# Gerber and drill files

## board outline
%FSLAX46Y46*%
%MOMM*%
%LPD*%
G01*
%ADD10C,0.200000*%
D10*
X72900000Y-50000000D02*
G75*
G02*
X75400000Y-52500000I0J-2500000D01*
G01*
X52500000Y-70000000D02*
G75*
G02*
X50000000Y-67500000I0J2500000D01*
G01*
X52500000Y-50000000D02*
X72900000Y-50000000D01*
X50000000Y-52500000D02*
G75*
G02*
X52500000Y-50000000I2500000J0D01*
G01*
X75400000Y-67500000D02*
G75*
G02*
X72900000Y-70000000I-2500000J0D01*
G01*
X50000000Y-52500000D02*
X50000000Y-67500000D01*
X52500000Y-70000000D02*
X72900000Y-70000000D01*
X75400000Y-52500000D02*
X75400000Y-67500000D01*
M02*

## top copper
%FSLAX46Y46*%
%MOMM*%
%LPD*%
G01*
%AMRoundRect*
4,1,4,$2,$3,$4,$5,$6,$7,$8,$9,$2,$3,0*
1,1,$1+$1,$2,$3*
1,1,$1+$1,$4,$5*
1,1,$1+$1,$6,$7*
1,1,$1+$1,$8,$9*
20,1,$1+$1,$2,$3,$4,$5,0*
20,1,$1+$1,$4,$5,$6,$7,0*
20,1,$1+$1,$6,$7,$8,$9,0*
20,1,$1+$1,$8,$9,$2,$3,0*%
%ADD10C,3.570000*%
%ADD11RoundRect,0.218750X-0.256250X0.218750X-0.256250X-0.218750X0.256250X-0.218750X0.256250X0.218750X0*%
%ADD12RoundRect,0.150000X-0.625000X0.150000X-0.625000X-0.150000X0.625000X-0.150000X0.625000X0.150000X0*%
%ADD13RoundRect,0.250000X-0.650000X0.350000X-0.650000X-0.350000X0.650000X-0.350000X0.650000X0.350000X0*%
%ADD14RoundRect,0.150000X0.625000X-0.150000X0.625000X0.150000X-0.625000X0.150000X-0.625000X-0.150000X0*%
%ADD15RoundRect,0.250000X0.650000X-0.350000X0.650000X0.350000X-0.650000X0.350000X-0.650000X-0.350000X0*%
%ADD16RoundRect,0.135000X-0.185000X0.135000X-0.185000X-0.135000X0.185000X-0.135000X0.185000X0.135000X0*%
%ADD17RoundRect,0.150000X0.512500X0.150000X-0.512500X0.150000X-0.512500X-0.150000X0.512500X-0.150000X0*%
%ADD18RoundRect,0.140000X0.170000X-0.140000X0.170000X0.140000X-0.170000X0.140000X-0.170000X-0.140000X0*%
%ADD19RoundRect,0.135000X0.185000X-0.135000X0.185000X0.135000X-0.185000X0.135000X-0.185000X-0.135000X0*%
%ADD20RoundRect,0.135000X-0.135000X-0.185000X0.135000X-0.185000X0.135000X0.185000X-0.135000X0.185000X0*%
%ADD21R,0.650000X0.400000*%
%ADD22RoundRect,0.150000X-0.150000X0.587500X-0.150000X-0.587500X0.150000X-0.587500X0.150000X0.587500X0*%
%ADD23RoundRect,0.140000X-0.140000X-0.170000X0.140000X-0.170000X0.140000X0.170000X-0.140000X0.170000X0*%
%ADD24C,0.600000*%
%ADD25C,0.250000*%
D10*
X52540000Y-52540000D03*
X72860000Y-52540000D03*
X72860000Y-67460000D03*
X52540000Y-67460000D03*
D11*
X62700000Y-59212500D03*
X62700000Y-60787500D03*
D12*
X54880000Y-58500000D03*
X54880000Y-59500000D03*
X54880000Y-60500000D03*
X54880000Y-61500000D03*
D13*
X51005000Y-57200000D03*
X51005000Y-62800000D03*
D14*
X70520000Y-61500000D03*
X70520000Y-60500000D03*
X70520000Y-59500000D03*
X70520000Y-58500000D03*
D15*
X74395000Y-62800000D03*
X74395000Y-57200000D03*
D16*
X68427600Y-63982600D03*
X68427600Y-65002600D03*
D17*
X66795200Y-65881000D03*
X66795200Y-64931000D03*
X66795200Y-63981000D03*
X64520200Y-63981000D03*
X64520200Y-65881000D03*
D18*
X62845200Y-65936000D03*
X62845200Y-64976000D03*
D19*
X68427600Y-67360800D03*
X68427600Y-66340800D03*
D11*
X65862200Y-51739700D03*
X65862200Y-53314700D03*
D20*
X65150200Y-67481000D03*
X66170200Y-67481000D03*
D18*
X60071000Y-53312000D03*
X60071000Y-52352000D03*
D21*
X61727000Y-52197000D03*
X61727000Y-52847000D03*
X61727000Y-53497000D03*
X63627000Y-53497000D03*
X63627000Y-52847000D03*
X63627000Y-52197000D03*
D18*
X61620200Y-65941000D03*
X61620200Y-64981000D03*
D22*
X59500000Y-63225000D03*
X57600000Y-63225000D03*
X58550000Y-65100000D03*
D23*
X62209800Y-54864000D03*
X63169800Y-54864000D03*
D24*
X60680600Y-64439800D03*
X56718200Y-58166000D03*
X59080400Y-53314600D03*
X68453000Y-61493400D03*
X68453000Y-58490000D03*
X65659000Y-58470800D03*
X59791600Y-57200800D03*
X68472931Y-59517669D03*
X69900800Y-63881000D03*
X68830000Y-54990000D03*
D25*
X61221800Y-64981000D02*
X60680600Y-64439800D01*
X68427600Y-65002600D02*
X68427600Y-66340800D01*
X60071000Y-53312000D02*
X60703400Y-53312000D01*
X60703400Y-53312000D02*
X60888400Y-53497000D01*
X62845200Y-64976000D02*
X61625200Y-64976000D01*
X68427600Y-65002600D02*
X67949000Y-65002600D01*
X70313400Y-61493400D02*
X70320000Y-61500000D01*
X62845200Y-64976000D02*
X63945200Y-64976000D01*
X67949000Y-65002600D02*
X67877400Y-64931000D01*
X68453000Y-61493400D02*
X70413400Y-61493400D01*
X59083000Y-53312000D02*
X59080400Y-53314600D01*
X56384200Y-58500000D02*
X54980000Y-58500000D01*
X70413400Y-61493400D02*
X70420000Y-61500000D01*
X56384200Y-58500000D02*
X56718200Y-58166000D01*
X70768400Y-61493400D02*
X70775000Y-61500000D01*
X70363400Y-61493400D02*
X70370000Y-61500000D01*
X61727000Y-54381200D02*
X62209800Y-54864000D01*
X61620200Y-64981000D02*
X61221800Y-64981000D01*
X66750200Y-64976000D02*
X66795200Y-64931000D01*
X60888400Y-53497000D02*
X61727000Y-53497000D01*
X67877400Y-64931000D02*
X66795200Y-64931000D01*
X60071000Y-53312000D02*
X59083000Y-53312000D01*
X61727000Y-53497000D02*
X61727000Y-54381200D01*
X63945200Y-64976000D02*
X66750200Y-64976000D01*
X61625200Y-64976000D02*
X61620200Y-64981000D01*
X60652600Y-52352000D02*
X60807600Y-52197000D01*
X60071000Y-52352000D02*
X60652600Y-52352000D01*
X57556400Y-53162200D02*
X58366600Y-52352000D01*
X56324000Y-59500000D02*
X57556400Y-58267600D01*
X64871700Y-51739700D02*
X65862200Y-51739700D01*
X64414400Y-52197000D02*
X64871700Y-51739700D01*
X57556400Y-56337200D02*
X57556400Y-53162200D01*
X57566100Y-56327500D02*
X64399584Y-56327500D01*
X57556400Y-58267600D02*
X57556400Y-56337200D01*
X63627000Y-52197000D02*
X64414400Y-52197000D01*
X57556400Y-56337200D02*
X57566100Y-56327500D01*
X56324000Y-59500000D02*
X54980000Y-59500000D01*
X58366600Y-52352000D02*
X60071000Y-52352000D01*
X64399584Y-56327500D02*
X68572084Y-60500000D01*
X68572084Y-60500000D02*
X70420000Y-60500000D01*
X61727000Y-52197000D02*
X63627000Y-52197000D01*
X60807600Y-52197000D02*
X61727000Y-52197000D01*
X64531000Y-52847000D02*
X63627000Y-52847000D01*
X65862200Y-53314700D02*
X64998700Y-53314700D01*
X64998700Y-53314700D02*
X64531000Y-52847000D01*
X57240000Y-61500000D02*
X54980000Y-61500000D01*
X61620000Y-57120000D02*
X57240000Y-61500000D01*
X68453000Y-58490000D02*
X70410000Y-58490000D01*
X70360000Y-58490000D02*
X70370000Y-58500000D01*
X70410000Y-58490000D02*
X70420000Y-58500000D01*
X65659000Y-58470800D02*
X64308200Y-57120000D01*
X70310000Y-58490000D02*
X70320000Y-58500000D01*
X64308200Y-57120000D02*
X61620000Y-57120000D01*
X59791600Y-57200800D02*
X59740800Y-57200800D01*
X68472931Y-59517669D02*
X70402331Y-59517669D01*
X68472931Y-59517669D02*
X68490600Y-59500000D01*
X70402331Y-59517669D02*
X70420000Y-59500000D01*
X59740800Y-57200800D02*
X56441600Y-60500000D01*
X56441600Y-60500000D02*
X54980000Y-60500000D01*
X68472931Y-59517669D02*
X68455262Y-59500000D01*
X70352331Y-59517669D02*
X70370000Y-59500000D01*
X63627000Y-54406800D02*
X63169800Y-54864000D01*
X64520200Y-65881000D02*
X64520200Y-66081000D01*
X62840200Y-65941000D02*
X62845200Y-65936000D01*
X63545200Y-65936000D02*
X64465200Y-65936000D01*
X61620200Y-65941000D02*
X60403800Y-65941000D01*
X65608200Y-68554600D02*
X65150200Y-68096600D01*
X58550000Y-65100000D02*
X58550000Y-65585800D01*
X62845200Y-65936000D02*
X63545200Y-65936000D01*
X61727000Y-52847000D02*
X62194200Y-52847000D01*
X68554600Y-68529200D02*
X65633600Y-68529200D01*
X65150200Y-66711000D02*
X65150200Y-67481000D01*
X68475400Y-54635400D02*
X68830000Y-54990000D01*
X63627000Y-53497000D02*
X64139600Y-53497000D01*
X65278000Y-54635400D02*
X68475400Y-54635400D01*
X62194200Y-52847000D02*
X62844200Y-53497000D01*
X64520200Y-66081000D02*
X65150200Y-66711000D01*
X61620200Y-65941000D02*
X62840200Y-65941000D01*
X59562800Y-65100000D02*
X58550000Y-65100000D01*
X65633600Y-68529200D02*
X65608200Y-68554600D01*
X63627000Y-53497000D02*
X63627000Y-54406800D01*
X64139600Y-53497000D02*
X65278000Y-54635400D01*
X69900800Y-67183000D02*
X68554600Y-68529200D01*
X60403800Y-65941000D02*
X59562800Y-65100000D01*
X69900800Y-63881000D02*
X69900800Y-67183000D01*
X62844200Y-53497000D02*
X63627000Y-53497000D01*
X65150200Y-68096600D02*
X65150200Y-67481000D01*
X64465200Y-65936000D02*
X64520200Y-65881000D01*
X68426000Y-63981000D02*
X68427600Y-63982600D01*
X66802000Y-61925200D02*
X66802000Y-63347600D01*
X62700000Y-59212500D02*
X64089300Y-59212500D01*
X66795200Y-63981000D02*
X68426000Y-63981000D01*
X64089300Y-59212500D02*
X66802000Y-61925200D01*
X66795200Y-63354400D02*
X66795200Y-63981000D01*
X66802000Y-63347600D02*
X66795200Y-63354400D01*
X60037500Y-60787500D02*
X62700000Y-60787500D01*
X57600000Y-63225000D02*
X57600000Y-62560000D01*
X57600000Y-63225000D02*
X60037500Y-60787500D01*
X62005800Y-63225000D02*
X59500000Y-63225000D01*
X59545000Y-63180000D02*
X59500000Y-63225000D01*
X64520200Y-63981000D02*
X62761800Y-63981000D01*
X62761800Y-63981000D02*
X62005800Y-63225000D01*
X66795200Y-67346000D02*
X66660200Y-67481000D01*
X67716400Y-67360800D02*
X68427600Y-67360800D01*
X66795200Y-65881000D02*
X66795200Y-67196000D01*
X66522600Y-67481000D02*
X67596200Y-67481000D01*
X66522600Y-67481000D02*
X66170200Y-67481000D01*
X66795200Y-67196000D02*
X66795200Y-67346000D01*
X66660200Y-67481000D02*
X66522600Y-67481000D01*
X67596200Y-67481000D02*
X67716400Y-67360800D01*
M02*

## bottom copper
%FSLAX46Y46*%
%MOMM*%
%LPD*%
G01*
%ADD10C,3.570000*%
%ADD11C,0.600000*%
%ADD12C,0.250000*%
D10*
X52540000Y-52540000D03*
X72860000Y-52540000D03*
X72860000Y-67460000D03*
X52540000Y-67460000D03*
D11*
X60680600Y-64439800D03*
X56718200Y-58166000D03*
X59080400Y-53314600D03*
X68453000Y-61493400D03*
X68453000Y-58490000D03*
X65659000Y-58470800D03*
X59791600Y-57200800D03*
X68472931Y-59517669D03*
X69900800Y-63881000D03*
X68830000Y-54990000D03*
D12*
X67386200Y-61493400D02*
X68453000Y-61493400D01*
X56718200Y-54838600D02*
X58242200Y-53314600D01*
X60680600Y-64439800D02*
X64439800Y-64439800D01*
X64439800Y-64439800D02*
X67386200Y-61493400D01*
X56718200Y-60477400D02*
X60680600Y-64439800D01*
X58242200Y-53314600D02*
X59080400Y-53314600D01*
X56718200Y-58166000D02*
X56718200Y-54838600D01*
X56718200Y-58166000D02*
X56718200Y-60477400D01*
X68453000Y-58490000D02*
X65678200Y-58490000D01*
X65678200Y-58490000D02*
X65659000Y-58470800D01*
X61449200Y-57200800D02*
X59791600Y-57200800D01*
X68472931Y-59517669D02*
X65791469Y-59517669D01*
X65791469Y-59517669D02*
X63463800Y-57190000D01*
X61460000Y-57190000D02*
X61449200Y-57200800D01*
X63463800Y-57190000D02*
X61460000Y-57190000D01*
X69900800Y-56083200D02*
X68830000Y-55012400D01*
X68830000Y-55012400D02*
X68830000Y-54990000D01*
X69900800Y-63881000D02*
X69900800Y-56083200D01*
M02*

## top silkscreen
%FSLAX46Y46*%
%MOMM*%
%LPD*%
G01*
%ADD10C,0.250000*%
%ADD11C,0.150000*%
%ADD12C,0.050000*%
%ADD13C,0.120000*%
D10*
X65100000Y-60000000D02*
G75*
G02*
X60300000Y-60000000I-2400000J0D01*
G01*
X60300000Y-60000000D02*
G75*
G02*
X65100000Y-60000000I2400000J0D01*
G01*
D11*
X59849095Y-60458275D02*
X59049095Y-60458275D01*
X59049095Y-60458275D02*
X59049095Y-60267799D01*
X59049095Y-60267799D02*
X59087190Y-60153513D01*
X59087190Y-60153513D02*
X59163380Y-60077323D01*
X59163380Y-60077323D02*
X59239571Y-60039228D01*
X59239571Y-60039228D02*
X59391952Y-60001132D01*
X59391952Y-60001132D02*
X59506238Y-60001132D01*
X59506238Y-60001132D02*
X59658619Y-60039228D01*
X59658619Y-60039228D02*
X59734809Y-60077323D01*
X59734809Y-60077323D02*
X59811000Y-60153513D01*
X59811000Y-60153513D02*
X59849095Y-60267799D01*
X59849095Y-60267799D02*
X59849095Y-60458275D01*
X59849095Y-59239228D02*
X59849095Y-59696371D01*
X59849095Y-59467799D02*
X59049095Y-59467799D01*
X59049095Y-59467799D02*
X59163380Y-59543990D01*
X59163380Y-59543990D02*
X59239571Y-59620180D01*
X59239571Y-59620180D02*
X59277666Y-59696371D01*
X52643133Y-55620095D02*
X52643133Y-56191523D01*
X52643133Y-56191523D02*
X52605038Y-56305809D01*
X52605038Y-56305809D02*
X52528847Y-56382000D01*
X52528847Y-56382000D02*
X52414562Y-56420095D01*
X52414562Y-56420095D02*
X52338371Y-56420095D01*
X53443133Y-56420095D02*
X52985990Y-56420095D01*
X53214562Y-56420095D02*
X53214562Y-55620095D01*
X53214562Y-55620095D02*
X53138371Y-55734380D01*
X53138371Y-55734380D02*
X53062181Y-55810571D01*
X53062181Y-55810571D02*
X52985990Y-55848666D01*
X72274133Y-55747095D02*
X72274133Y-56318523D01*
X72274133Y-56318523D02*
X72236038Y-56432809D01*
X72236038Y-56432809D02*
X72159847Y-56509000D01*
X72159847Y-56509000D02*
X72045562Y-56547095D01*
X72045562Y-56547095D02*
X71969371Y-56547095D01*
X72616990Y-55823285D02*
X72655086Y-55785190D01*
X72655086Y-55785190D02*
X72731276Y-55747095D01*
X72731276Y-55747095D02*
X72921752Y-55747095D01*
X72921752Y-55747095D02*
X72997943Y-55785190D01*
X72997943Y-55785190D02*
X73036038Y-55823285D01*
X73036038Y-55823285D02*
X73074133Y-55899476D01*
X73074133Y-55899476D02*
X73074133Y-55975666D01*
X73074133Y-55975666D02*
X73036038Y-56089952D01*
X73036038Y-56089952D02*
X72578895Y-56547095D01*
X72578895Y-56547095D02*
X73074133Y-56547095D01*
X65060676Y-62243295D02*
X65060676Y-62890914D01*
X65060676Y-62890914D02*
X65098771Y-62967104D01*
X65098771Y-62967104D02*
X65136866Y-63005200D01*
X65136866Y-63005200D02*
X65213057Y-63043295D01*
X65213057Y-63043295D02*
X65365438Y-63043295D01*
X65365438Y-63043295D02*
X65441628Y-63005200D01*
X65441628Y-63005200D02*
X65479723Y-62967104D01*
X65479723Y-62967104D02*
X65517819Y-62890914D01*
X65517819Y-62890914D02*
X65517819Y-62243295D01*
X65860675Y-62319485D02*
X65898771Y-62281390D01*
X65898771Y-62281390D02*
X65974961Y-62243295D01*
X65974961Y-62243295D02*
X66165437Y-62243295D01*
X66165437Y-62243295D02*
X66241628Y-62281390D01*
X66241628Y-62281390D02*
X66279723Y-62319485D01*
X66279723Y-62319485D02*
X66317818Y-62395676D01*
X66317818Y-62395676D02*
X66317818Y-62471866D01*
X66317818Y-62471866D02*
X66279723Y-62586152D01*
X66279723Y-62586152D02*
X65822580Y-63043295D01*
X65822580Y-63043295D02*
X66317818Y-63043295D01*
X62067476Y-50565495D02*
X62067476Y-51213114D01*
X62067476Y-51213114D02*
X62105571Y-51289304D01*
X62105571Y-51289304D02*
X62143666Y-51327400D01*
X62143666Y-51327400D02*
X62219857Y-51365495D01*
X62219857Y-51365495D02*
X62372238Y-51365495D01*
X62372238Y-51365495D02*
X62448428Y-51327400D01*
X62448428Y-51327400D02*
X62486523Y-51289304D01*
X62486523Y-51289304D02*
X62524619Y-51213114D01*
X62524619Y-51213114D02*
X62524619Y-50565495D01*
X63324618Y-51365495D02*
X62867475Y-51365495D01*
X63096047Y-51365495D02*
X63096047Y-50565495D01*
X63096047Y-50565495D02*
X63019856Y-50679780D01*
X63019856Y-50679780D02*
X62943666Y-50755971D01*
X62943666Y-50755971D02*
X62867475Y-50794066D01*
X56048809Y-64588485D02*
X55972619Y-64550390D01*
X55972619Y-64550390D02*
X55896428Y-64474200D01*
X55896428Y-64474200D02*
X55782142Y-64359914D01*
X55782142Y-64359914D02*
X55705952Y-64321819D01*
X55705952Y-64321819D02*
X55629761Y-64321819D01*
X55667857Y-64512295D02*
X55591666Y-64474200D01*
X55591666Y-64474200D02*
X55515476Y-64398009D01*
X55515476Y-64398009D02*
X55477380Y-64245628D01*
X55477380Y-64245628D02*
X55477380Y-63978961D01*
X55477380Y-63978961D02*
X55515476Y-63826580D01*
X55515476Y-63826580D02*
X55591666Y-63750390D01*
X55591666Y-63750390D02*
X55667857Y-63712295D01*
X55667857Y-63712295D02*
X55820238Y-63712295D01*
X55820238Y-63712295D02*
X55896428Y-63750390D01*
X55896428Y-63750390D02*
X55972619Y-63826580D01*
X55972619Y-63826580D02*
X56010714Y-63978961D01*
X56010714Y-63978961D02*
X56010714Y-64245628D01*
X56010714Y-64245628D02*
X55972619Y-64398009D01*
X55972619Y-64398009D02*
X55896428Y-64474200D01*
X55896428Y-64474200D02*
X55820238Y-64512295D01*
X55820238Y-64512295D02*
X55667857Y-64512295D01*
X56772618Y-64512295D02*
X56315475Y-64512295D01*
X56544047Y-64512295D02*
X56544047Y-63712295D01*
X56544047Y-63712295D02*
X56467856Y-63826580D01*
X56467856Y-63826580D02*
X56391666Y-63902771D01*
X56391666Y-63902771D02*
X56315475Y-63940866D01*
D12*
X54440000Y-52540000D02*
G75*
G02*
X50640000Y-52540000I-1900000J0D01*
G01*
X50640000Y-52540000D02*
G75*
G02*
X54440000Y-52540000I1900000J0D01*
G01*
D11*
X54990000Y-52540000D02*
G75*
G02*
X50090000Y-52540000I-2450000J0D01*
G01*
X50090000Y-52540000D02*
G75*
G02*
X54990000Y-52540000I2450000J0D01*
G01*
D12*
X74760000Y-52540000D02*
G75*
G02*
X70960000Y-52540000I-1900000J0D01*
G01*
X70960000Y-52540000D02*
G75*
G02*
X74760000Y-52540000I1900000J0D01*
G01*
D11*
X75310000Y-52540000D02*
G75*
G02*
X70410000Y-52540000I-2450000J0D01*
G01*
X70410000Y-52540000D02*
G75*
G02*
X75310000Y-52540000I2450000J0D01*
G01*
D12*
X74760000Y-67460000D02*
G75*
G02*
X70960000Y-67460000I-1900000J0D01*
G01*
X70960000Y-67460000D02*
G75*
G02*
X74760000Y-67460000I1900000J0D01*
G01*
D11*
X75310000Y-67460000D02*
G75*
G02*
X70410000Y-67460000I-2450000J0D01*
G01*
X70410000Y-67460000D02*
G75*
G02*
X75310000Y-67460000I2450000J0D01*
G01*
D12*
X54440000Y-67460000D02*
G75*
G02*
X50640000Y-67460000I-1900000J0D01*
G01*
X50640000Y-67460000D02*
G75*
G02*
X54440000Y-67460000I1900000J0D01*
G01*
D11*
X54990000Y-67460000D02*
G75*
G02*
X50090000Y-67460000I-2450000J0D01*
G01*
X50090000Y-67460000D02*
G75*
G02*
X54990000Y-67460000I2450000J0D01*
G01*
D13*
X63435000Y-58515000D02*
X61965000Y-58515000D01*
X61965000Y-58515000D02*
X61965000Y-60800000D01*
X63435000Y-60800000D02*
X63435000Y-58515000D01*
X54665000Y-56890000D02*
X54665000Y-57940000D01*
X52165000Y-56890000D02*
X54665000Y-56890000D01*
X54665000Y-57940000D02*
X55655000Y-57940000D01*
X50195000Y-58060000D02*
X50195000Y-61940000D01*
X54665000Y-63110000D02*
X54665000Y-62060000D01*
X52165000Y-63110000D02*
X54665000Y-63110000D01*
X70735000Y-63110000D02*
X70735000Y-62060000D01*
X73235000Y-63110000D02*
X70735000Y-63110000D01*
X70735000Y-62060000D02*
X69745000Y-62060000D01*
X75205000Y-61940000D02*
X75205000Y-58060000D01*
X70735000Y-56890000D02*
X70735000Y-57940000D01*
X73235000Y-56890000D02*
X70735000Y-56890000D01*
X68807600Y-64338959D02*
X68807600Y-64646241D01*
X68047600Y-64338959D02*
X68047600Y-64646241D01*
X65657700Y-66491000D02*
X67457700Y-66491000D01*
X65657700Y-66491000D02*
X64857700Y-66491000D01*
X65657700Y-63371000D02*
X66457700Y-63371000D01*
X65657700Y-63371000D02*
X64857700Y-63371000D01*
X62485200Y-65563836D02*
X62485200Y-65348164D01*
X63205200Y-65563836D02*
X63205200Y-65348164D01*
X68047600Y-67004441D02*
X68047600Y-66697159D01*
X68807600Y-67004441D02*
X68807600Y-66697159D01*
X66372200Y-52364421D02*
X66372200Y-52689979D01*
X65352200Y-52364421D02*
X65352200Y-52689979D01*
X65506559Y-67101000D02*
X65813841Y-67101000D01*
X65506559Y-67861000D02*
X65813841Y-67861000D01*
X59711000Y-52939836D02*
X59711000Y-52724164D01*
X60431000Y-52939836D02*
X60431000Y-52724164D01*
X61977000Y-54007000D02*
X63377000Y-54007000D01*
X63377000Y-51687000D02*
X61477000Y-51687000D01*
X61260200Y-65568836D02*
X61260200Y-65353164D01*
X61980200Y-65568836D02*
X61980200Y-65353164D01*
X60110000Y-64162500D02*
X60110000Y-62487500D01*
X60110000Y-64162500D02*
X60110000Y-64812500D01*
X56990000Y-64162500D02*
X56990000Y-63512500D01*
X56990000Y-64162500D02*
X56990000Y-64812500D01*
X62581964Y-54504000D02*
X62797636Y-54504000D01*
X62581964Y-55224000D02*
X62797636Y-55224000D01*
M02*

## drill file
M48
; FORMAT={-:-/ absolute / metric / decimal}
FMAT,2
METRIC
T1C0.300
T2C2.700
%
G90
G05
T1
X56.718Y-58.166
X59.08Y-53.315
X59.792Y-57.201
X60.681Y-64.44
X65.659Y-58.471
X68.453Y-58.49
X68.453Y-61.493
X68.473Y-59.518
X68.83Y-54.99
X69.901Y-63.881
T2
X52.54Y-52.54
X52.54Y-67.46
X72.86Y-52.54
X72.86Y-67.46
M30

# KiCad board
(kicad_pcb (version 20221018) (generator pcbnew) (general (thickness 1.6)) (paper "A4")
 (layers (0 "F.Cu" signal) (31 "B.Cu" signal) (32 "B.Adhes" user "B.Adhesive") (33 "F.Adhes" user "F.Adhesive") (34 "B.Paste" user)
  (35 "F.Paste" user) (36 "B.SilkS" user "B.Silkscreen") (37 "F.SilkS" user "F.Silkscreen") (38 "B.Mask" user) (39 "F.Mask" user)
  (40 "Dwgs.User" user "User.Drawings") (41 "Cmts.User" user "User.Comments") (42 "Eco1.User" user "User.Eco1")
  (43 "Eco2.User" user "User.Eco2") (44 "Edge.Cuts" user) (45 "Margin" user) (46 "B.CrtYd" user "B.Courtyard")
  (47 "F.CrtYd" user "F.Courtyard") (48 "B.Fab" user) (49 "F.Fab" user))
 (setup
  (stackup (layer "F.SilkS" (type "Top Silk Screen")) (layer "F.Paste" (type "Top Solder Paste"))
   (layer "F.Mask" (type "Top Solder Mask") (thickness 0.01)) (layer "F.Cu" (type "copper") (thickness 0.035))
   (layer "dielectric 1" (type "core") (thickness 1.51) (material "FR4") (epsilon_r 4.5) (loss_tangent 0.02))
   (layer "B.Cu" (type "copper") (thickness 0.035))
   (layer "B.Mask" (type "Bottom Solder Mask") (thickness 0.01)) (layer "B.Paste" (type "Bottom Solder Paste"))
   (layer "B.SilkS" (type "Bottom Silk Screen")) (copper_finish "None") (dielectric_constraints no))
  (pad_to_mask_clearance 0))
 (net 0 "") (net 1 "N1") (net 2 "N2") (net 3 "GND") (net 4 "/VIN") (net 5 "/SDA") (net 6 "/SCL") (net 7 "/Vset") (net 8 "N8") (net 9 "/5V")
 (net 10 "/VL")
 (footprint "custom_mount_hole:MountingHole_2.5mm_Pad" (layer "F.Cu") (at 52.54 52.54)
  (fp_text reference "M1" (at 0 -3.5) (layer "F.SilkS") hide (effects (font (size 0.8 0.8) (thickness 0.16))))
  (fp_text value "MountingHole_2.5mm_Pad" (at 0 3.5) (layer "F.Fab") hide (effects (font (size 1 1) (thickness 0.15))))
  (fp_circle (center 0 0) (end 1.9 0) (stroke (width 0.05) (type solid)) (fill none) (layer "F.SilkS"))
  (fp_circle (center 0 0) (end 2.45 0) (stroke (width 0.15) (type solid)) (fill none) (layer "F.SilkS"))
  (pad "~" thru_hole circle (at 0 0) (size 3.57 3.57) (drill 2.7) (layers "*.Cu" "*.Mask")))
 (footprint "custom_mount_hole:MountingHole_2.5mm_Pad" (layer "F.Cu") (at 72.86 52.54)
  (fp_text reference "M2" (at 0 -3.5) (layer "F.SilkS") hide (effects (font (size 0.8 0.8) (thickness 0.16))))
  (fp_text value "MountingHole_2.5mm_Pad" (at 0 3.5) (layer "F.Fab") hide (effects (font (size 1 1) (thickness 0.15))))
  (fp_circle (center 0 0) (end 1.9 0) (stroke (width 0.05) (type solid)) (fill none) (layer "F.SilkS"))
  (fp_circle (center 0 0) (end 2.45 0) (stroke (width 0.15) (type solid)) (fill none) (layer "F.SilkS"))
  (pad "~" thru_hole circle (at 0 0) (size 3.57 3.57) (drill 2.7) (layers "*.Cu" "*.Mask")))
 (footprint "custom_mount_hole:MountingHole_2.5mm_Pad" (layer "F.Cu") (at 72.86 67.46)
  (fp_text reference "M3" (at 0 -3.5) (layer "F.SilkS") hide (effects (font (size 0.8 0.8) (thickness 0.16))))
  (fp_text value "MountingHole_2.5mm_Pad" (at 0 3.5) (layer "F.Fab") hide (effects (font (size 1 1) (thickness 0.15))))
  (fp_circle (center 0 0) (end 1.9 0) (stroke (width 0.05) (type solid)) (fill none) (layer "F.SilkS"))
  (fp_circle (center 0 0) (end 2.45 0) (stroke (width 0.15) (type solid)) (fill none) (layer "F.SilkS"))
  (pad "~" thru_hole circle (at 0 0) (size 3.57 3.57) (drill 2.7) (layers "*.Cu" "*.Mask")))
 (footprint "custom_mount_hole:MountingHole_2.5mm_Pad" (layer "F.Cu") (at 52.54 67.46)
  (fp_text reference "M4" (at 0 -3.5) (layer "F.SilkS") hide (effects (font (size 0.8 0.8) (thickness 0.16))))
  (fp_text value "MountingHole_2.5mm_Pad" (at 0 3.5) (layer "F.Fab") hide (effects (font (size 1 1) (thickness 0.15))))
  (fp_circle (center 0 0) (end 1.9 0) (stroke (width 0.05) (type solid)) (fill none) (layer "F.SilkS"))
  (fp_circle (center 0 0) (end 2.45 0) (stroke (width 0.15) (type solid)) (fill none) (layer "F.SilkS"))
  (pad "~" thru_hole circle (at 0 0) (size 3.57 3.57) (drill 2.7) (layers "*.Cu" "*.Mask")))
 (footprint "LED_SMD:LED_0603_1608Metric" (layer "F.Cu") (at 62.7 60 -90)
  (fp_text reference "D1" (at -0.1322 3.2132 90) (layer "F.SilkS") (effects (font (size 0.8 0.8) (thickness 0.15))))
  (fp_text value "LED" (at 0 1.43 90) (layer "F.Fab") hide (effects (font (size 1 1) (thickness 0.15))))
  (fp_line (start -1.485 -0.735) (end -1.485 0.735) (stroke (width 0.12) (type solid)) (layer "F.SilkS"))
  (fp_line (start -1.485 0.735) (end 0.8 0.735) (stroke (width 0.12) (type solid)) (layer "F.SilkS"))
  (fp_line (start 0.8 -0.735) (end -1.485 -0.735) (stroke (width 0.12) (type solid)) (layer "F.SilkS"))
  (pad "1" smd roundrect (at -0.7875 0 270) (size 0.875 0.95) (layers "F.Cu" "F.Paste" "F.Mask") (roundrect_rratio 0.25) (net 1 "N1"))
  (pad "2" smd roundrect (at 0.7875 0 270) (size 0.875 0.95) (layers "F.Cu" "F.Paste" "F.Mask") (roundrect_rratio 0.25) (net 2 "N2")))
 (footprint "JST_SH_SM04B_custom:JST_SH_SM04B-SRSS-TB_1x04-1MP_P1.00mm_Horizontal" (layer "F.Cu") (at 52.88 60 -90)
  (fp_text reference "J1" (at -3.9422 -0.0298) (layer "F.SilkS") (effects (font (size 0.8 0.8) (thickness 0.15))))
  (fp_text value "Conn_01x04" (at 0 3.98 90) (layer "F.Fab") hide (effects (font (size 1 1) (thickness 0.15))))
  (fp_line (start -3.11 -1.785) (end -2.06 -1.785) (stroke (width 0.12) (type solid)) (layer "F.SilkS"))
  (fp_line (start -3.11 0.715) (end -3.11 -1.785) (stroke (width 0.12) (type solid)) (layer "F.SilkS"))
  (fp_line (start -2.06 -1.785) (end -2.06 -2.775) (stroke (width 0.12) (type solid)) (layer "F.SilkS"))
  (fp_line (start -1.94 2.685) (end 1.94 2.685) (stroke (width 0.12) (type solid)) (layer "F.SilkS"))
  (fp_line (start 3.11 -1.785) (end 2.06 -1.785) (stroke (width 0.12) (type solid)) (layer "F.SilkS"))
  (fp_line (start 3.11 0.715) (end 3.11 -1.785) (stroke (width 0.12) (type solid)) (layer "F.SilkS"))
  (pad "1" smd roundrect (at -1.5 -2 270) (size 0.6 1.55) (layers "F.Cu" "F.Paste" "F.Mask") (roundrect_rratio 0.25) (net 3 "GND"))
  (pad "2" smd roundrect (at -0.5 -2 270) (size 0.6 1.55) (layers "F.Cu" "F.Paste" "F.Mask") (roundrect_rratio 0.25) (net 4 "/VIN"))
  (pad "3" smd roundrect (at 0.5 -2 270) (size 0.6 1.55) (layers "F.Cu" "F.Paste" "F.Mask") (roundrect_rratio 0.25) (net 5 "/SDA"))
  (pad "4" smd roundrect (at 1.5 -2 270) (size 0.6 1.55) (layers "F.Cu" "F.Paste" "F.Mask") (roundrect_rratio 0.25) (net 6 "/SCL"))
  (pad "MP" smd roundrect (at -2.8 1.875 270) (size 1.2 1.8) (layers "F.Cu" "F.Paste" "F.Mask") (roundrect_rratio 0.2083333333))
  (pad "MP" smd roundrect (at 2.8 1.875 270) (size 1.2 1.8) (layers "F.Cu" "F.Paste" "F.Mask") (roundrect_rratio 0.2083333333)))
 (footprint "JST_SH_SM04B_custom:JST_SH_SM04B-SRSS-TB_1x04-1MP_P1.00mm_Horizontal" (layer "F.Cu") (at 72.52 60 90)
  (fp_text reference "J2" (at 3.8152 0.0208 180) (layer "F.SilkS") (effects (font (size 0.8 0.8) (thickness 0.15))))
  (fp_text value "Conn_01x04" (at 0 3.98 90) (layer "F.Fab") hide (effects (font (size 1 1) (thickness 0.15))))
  (fp_line (start -3.11 -1.785) (end -2.06 -1.785) (stroke (width 0.12) (type solid)) (layer "F.SilkS"))
  (fp_line (start -3.11 0.715) (end -3.11 -1.785) (stroke (width 0.12) (type solid)) (layer "F.SilkS"))
  (fp_line (start -2.06 -1.785) (end -2.06 -2.775) (stroke (width 0.12) (type solid)) (layer "F.SilkS"))
  (fp_line (start -1.94 2.685) (end 1.94 2.685) (stroke (width 0.12) (type solid)) (layer "F.SilkS"))
  (fp_line (start 3.11 -1.785) (end 2.06 -1.785) (stroke (width 0.12) (type solid)) (layer "F.SilkS"))
  (fp_line (start 3.11 0.715) (end 3.11 -1.785) (stroke (width 0.12) (type solid)) (layer "F.SilkS"))
  (pad "1" smd roundrect (at -1.5 -2 90) (size 0.6 1.55) (layers "F.Cu" "F.Paste" "F.Mask") (roundrect_rratio 0.25) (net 3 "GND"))
  (pad "2" smd roundrect (at -0.5 -2 90) (size 0.6 1.55) (layers "F.Cu" "F.Paste" "F.Mask") (roundrect_rratio 0.25) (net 4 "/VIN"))
  (pad "3" smd roundrect (at 0.5 -2 90) (size 0.6 1.55) (layers "F.Cu" "F.Paste" "F.Mask") (roundrect_rratio 0.25) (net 5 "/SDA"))
  (pad "4" smd roundrect (at 1.5 -2 90) (size 0.6 1.55) (layers "F.Cu" "F.Paste" "F.Mask") (roundrect_rratio 0.25) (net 6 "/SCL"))
  (pad "MP" smd roundrect (at -2.8 1.875 90) (size 1.2 1.8) (layers "F.Cu" "F.Paste" "F.Mask") (roundrect_rratio 0.2083333333))
  (pad "MP" smd roundrect (at 2.8 1.875 90) (size 1.2 1.8) (layers "F.Cu" "F.Paste" "F.Mask") (roundrect_rratio 0.2083333333)))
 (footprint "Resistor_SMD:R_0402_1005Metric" (layer "F.Cu") (at 68.4276 64.4926 -90)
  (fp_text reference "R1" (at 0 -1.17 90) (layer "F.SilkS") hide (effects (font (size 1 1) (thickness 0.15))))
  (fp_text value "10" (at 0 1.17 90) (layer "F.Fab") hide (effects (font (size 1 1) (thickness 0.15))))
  (fp_line (start -0.153641 -0.38) (end 0.153641 -0.38) (stroke (width 0.12) (type solid)) (layer "F.SilkS"))
  (fp_line (start -0.153641 0.38) (end 0.153641 0.38) (stroke (width 0.12) (type solid)) (layer "F.SilkS"))
  (pad "1" smd roundrect (at -0.51 0 270) (size 0.54 0.64) (layers "F.Cu" "F.Paste" "F.Mask") (roundrect_rratio 0.25) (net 1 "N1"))
  (pad "2" smd roundrect (at 0.51 0 270) (size 0.54 0.64) (layers "F.Cu" "F.Paste" "F.Mask") (roundrect_rratio 0.25) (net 3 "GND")))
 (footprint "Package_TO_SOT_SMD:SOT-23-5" (layer "F.Cu") (at 65.6577 64.931 180)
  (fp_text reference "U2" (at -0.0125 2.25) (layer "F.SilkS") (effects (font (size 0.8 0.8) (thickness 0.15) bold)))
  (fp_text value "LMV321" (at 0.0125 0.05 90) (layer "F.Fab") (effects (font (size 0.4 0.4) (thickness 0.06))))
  (fp_line (start 0 -1.56) (end -1.8 -1.56) (stroke (width 0.12) (type solid)) (layer "F.SilkS"))
  (fp_line (start 0 -1.56) (end 0.8 -1.56) (stroke (width 0.12) (type solid)) (layer "F.SilkS"))
  (fp_line (start 0 1.56) (end -0.8 1.56) (stroke (width 0.12) (type solid)) (layer "F.SilkS"))
  (fp_line (start 0 1.56) (end 0.8 1.56) (stroke (width 0.12) (type solid)) (layer "F.SilkS"))
  (pad "1" smd roundrect (at -1.1375 -0.95 180) (size 1.325 0.6) (layers "F.Cu" "F.Paste" "F.Mask") (roundrect_rratio 0.25) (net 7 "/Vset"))
  (pad "2" smd roundrect (at -1.1375 0 180) (size 1.325 0.6) (layers "F.Cu" "F.Paste" "F.Mask") (roundrect_rratio 0.25) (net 3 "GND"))
  (pad "3" smd roundrect (at -1.1375 0.95 180) (size 1.325 0.6) (layers "F.Cu" "F.Paste" "F.Mask") (roundrect_rratio 0.25) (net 1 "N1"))
  (pad "4" smd roundrect (at 1.1375 0.95 180) (size 1.325 0.6) (layers "F.Cu" "F.Paste" "F.Mask") (roundrect_rratio 0.25) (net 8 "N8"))
  (pad "5" smd roundrect (at 1.1375 -0.95 180) (size 1.325 0.6) (layers "F.Cu" "F.Paste" "F.Mask") (roundrect_rratio 0.25) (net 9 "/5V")))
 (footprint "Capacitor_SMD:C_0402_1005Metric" (layer "F.Cu") (at 62.8452 65.456 90)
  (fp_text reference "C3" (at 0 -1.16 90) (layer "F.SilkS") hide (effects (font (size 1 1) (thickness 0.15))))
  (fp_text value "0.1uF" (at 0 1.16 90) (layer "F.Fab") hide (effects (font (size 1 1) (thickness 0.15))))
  (fp_line (start -0.107836 -0.36) (end 0.107836 -0.36) (stroke (width 0.12) (type solid)) (layer "F.SilkS"))
  (fp_line (start -0.107836 0.36) (end 0.107836 0.36) (stroke (width 0.12) (type solid)) (layer "F.SilkS"))
  (pad "1" smd roundrect (at -0.48 0 90) (size 0.56 0.62) (layers "F.Cu" "F.Paste" "F.Mask") (roundrect_rratio 0.25) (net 9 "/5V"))
  (pad "2" smd roundrect (at 0.48 0 90) (size 0.56 0.62) (layers "F.Cu" "F.Paste" "F.Mask") (roundrect_rratio 0.25) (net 3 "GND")))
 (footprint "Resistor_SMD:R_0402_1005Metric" (layer "F.Cu") (at 68.4276 66.8508 90)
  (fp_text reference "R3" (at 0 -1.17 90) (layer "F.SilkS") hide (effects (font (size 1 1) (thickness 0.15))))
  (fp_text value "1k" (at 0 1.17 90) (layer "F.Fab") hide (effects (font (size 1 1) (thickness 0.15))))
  (fp_line (start -0.153641 -0.38) (end 0.153641 -0.38) (stroke (width 0.12) (type solid)) (layer "F.SilkS"))
  (fp_line (start -0.153641 0.38) (end 0.153641 0.38) (stroke (width 0.12) (type solid)) (layer "F.SilkS"))
  (pad "1" smd roundrect (at -0.51 0 90) (size 0.54 0.64) (layers "F.Cu" "F.Paste" "F.Mask") (roundrect_rratio 0.25) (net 7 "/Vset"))
  (pad "2" smd roundrect (at 0.51 0 90) (size 0.54 0.64) (layers "F.Cu" "F.Paste" "F.Mask") (roundrect_rratio 0.25) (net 3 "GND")))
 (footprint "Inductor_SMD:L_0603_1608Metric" (layer "F.Cu") (at 65.8622 52.5272 -90)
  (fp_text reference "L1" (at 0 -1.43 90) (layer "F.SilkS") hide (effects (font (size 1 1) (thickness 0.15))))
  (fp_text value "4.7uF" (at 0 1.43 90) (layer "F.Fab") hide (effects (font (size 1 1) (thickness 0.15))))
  (fp_line (start -0.162779 -0.51) (end 0.162779 -0.51) (stroke (width 0.12) (type solid)) (layer "F.SilkS"))
  (fp_line (start -0.162779 0.51) (end 0.162779 0.51) (stroke (width 0.12) (type solid)) (layer "F.SilkS"))
  (pad "1" smd roundrect (at -0.7875 0 270) (size 0.875 0.95) (layers "F.Cu" "F.Paste" "F.Mask") (roundrect_rratio 0.25) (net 4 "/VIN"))
  (pad "2" smd roundrect (at 0.7875 0 270) (size 0.875 0.95) (layers "F.Cu" "F.Paste" "F.Mask") (roundrect_rratio 0.25) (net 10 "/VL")))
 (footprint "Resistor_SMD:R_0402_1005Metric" (layer "F.Cu") (at 65.6602 67.481)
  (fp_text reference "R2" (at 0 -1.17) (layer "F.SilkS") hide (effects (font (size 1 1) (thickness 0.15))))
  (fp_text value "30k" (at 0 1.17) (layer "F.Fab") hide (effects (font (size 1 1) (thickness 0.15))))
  (fp_line (start -0.153641 -0.38) (end 0.153641 -0.38) (stroke (width 0.12) (type solid)) (layer "F.SilkS"))
  (fp_line (start -0.153641 0.38) (end 0.153641 0.38) (stroke (width 0.12) (type solid)) (layer "F.SilkS"))
  (pad "1" smd roundrect (at -0.51 0) (size 0.54 0.64) (layers "F.Cu" "F.Paste" "F.Mask") (roundrect_rratio 0.25) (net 9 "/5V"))
  (pad "2" smd roundrect (at 0.51 0) (size 0.54 0.64) (layers "F.Cu" "F.Paste" "F.Mask") (roundrect_rratio 0.25) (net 7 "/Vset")))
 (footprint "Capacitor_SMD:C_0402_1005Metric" (layer "F.Cu") (at 60.071 52.832 90)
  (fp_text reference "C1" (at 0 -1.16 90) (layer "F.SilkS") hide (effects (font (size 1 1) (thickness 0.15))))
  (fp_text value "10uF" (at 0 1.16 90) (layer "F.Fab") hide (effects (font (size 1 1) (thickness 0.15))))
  (fp_line (start -0.107836 -0.36) (end 0.107836 -0.36) (stroke (width 0.12) (type solid)) (layer "F.SilkS"))
  (fp_line (start -0.107836 0.36) (end 0.107836 0.36) (stroke (width 0.12) (type solid)) (layer "F.SilkS"))
  (pad "1" smd roundrect (at -0.48 0 90) (size 0.56 0.62) (layers "F.Cu" "F.Paste" "F.Mask") (roundrect_rratio 0.25) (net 3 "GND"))
  (pad "2" smd roundrect (at 0.48 0 90) (size 0.56 0.62) (layers "F.Cu" "F.Paste" "F.Mask") (roundrect_rratio 0.25) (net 4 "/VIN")))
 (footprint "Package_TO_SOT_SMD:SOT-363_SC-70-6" (layer "F.Cu") (at 62.677 52.847)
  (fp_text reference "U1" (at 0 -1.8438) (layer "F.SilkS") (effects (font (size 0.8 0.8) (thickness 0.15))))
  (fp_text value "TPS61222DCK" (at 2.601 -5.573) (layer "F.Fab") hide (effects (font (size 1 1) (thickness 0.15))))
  (fp_line (start -0.7 1.16) (end 0.7 1.16) (stroke (width 0.12) (type solid)) (layer "F.SilkS"))
  (fp_line (start 0.7 -1.16) (end -1.2 -1.16) (stroke (width 0.12) (type solid)) (layer "F.SilkS"))
  (pad "1" smd rect (at -0.95 -0.65) (size 0.65 0.4) (layers "F.Cu" "F.Paste" "F.Mask") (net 4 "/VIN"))
  (pad "2" smd rect (at -0.95 0) (size 0.65 0.4) (layers "F.Cu" "F.Paste" "F.Mask") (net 9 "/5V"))
  (pad "3" smd rect (at -0.95 0.65) (size 0.65 0.4) (layers "F.Cu" "F.Paste" "F.Mask") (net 3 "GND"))
  (pad "4" smd rect (at 0.95 0.65) (size 0.65 0.4) (layers "F.Cu" "F.Paste" "F.Mask") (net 9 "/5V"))
  (pad "5" smd rect (at 0.95 0) (size 0.65 0.4) (layers "F.Cu" "F.Paste" "F.Mask") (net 10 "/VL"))
  (pad "6" smd rect (at 0.95 -0.65) (size 0.65 0.4) (layers "F.Cu" "F.Paste" "F.Mask") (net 4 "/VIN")))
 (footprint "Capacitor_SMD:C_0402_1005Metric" (layer "F.Cu") (at 61.6202 65.461 90)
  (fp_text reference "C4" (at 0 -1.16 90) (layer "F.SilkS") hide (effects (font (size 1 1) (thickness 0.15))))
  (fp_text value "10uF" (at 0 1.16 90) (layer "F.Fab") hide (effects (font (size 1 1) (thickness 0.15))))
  (fp_line (start -0.107836 -0.36) (end 0.107836 -0.36) (stroke (width 0.12) (type solid)) (layer "F.SilkS"))
  (fp_line (start -0.107836 0.36) (end 0.107836 0.36) (stroke (width 0.12) (type solid)) (layer "F.SilkS"))
  (pad "1" smd roundrect (at -0.48 0 90) (size 0.56 0.62) (layers "F.Cu" "F.Paste" "F.Mask") (roundrect_rratio 0.25) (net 9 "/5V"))
  (pad "2" smd roundrect (at 0.48 0 90) (size 0.56 0.62) (layers "F.Cu" "F.Paste" "F.Mask") (roundrect_rratio 0.25) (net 3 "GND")))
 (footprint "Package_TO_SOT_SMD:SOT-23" (layer "F.Cu") (at 58.55 64.1625 -90)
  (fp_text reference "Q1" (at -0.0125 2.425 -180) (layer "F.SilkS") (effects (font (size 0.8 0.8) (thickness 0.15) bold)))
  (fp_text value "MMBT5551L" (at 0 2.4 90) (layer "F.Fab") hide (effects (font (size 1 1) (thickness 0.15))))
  (fp_line (start 0 -1.56) (end -1.675 -1.56) (stroke (width 0.12) (type solid)) (layer "F.SilkS"))
  (fp_line (start 0 -1.56) (end 0.65 -1.56) (stroke (width 0.12) (type solid)) (layer "F.SilkS"))
  (fp_line (start 0 1.56) (end -0.65 1.56) (stroke (width 0.12) (type solid)) (layer "F.SilkS"))
  (fp_line (start 0 1.56) (end 0.65 1.56) (stroke (width 0.12) (type solid)) (layer "F.SilkS"))
  (pad "1" smd roundrect (at -0.9375 -0.95 270) (size 1.475 0.6) (layers "F.Cu" "F.Paste" "F.Mask") (roundrect_rratio 0.25) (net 8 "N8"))
  (pad "2" smd roundrect (at -0.9375 0.95 270) (size 1.475 0.6) (layers "F.Cu" "F.Paste" "F.Mask") (roundrect_rratio 0.25) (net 2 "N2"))
  (pad "3" smd roundrect (at 0.9375 0 270) (size 1.475 0.6) (layers "F.Cu" "F.Paste" "F.Mask") (roundrect_rratio 0.25) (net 9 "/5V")))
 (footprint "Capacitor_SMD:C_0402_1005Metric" (layer "F.Cu") (at 62.6898 54.864)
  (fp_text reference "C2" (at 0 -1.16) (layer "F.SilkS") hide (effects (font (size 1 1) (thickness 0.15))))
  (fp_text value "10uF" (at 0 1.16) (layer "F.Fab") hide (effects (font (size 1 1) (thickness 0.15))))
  (fp_line (start -0.107836 -0.36) (end 0.107836 -0.36) (stroke (width 0.12) (type solid)) (layer "F.SilkS"))
  (fp_line (start -0.107836 0.36) (end 0.107836 0.36) (stroke (width 0.12) (type solid)) (layer "F.SilkS"))
  (pad "1" smd roundrect (at -0.48 0) (size 0.56 0.62) (layers "F.Cu" "F.Paste" "F.Mask") (roundrect_rratio 0.25) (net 3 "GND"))
  (pad "2" smd roundrect (at 0.48 0) (size 0.56 0.62) (layers "F.Cu" "F.Paste" "F.Mask") (roundrect_rratio 0.25) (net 9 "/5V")))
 (gr_circle (center 62.7 60) (end 65.1 60) (stroke (width 0.25) (type solid)) (fill none) (layer "F.SilkS"))
 (gr_arc (start 72.9 50) (mid 74.667767 50.732233) (end 75.4 52.5) (stroke (width 0.2) (type solid)) (layer "Edge.Cuts"))
 (gr_arc (start 52.5 70) (mid 50.732233 69.267767) (end 50 67.5) (stroke (width 0.2) (type solid)) (layer "Edge.Cuts"))
 (gr_line (start 52.5 50) (end 72.9 50) (stroke (width 0.2) (type solid)) (layer "Edge.Cuts"))
 (gr_arc (start 50 52.5) (mid 50.732233 50.732233) (end 52.5 50) (stroke (width 0.2) (type solid)) (layer "Edge.Cuts"))
 (gr_arc (start 75.4 67.5) (mid 74.667767 69.267767) (end 72.9 70) (stroke (width 0.2) (type solid)) (layer "Edge.Cuts"))
 (gr_line (start 50 52.5) (end 50 67.5) (stroke (width 0.2) (type solid)) (layer "Edge.Cuts"))
 (gr_line (start 52.5 70) (end 72.9 70) (stroke (width 0.2) (type solid)) (layer "Edge.Cuts"))
 (gr_line (start 75.4 52.5) (end 75.4 67.5) (stroke (width 0.2) (type solid)) (layer "Edge.Cuts"))
 (segment (start 61.2218 64.981) (end 60.6806 64.4398) (width 0.25) (layer "F.Cu") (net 3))
 (segment (start 68.4276 65.0026) (end 68.4276 66.3408) (width 0.25) (layer "F.Cu") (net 3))
 (segment (start 60.071 53.312) (end 60.7034 53.312) (width 0.25) (layer "F.Cu") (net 3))
 (segment (start 60.7034 53.312) (end 60.8884 53.497) (width 0.25) (layer "F.Cu") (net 3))
 (segment (start 62.8452 64.976) (end 61.6252 64.976) (width 0.25) (layer "F.Cu") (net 3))
 (segment (start 68.4276 65.0026) (end 67.949 65.0026) (width 0.25) (layer "F.Cu") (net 3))
 (segment (start 70.3134 61.4934) (end 70.32 61.5) (width 0.25) (layer "F.Cu") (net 3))
 (segment (start 62.8452 64.976) (end 63.9452 64.976) (width 0.25) (layer "F.Cu") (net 3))
 (segment (start 67.949 65.0026) (end 67.8774 64.931) (width 0.25) (layer "F.Cu") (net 3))
 (segment (start 68.453 61.4934) (end 70.4134 61.4934) (width 0.25) (layer "F.Cu") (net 3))
 (segment (start 59.083 53.312) (end 59.0804 53.3146) (width 0.25) (layer "F.Cu") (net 3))
 (segment (start 56.3842 58.5) (end 54.98 58.5) (width 0.25) (layer "F.Cu") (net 3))
 (segment (start 70.4134 61.4934) (end 70.42 61.5) (width 0.25) (layer "F.Cu") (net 3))
 (segment (start 56.3842 58.5) (end 56.7182 58.166) (width 0.25) (layer "F.Cu") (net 3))
 (segment (start 70.7684 61.4934) (end 70.775 61.5) (width 0.25) (layer "F.Cu") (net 3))
 (segment (start 70.3634 61.4934) (end 70.37 61.5) (width 0.25) (layer "F.Cu") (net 3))
 (segment (start 61.727 54.3812) (end 62.2098 54.864) (width 0.25) (layer "F.Cu") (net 3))
 (segment (start 61.6202 64.981) (end 61.2218 64.981) (width 0.25) (layer "F.Cu") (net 3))
 (segment (start 66.7502 64.976) (end 66.7952 64.931) (width 0.25) (layer "F.Cu") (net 3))
 (segment (start 60.8884 53.497) (end 61.727 53.497) (width 0.25) (layer "F.Cu") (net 3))
 (segment (start 67.8774 64.931) (end 66.7952 64.931) (width 0.25) (layer "F.Cu") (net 3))
 (segment (start 60.071 53.312) (end 59.083 53.312) (width 0.25) (layer "F.Cu") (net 3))
 (segment (start 61.727 53.497) (end 61.727 54.3812) (width 0.25) (layer "F.Cu") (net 3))
 (segment (start 63.9452 64.976) (end 66.7502 64.976) (width 0.25) (layer "F.Cu") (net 3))
 (segment (start 61.6252 64.976) (end 61.6202 64.981) (width 0.25) (layer "F.Cu") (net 3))
 (via (at 60.6806 64.4398) (size 0.6) (drill 0.3) (layers "F.Cu" "B.Cu") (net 3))
 (via (at 56.7182 58.166) (size 0.6) (drill 0.3) (layers "F.Cu" "B.Cu") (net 3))
 (via (at 59.0804 53.3146) (size 0.6) (drill 0.3) (layers "F.Cu" "B.Cu") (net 3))
 (via (at 68.453 61.4934) (size 0.6) (drill 0.3) (layers "F.Cu" "B.Cu") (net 3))
 (segment (start 67.3862 61.4934) (end 68.453 61.4934) (width 0.25) (layer "B.Cu") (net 3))
 (segment (start 56.7182 54.8386) (end 58.2422 53.3146) (width 0.25) (layer "B.Cu") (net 3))
 (segment (start 60.6806 64.4398) (end 64.4398 64.4398) (width 0.25) (layer "B.Cu") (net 3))
 (segment (start 64.4398 64.4398) (end 67.3862 61.4934) (width 0.25) (layer "B.Cu") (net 3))
 (segment (start 56.7182 60.4774) (end 60.6806 64.4398) (width 0.25) (layer "B.Cu") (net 3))
 (segment (start 58.2422 53.3146) (end 59.0804 53.3146) (width 0.25) (layer "B.Cu") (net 3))
 (segment (start 56.7182 58.166) (end 56.7182 54.8386) (width 0.25) (layer "B.Cu") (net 3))
 (segment (start 56.7182 58.166) (end 56.7182 60.4774) (width 0.25) (layer "B.Cu") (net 3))
 (segment (start 60.6526 52.352) (end 60.8076 52.197) (width 0.25) (layer "F.Cu") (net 4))
 (segment (start 60.071 52.352) (end 60.6526 52.352) (width 0.25) (layer "F.Cu") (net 4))
 (segment (start 57.5564 53.1622) (end 58.3666 52.352) (width 0.25) (layer "F.Cu") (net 4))
 (segment (start 56.324 59.5) (end 57.5564 58.2676) (width 0.25) (layer "F.Cu") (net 4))
 (segment (start 64.8717 51.7397) (end 65.8622 51.7397) (width 0.25) (layer "F.Cu") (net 4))
 (segment (start 64.4144 52.197) (end 64.8717 51.7397) (width 0.25) (layer "F.Cu") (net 4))
 (segment (start 57.5564 56.3372) (end 57.5564 53.1622) (width 0.25) (layer "F.Cu") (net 4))
 (segment (start 57.5661 56.3275) (end 64.399584 56.3275) (width 0.25) (layer "F.Cu") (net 4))
 (segment (start 57.5564 58.2676) (end 57.5564 56.3372) (width 0.25) (layer "F.Cu") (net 4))
 (segment (start 63.627 52.197) (end 64.4144 52.197) (width 0.25) (layer "F.Cu") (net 4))
 (segment (start 57.5564 56.3372) (end 57.5661 56.3275) (width 0.25) (layer "F.Cu") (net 4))
 (segment (start 56.324 59.5) (end 54.98 59.5) (width 0.25) (layer "F.Cu") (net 4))
 (segment (start 58.3666 52.352) (end 60.071 52.352) (width 0.25) (layer "F.Cu") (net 4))
 (segment (start 64.399584 56.3275) (end 68.572084 60.5) (width 0.25) (layer "F.Cu") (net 4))
 (segment (start 68.572084 60.5) (end 70.42 60.5) (width 0.25) (layer "F.Cu") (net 4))
 (segment (start 61.727 52.197) (end 63.627 52.197) (width 0.25) (layer "F.Cu") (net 4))
 (segment (start 60.8076 52.197) (end 61.727 52.197) (width 0.25) (layer "F.Cu") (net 4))
 (segment (start 64.531 52.847) (end 63.627 52.847) (width 0.25) (layer "F.Cu") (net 10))
 (segment (start 65.8622 53.3147) (end 64.9987 53.3147) (width 0.25) (layer "F.Cu") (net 10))
 (segment (start 64.9987 53.3147) (end 64.531 52.847) (width 0.25) (layer "F.Cu") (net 10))
 (segment (start 57.24 61.5) (end 54.98 61.5) (width 0.25) (layer "F.Cu") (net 6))
 (segment (start 61.62 57.12) (end 57.24 61.5) (width 0.25) (layer "F.Cu") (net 6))
 (segment (start 68.453 58.49) (end 70.41 58.49) (width 0.25) (layer "F.Cu") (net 6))
 (segment (start 70.36 58.49) (end 70.37 58.5) (width 0.25) (layer "F.Cu") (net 6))
 (segment (start 70.41 58.49) (end 70.42 58.5) (width 0.25) (layer "F.Cu") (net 6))
 (segment (start 65.659 58.4708) (end 64.3082 57.12) (width 0.25) (layer "F.Cu") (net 6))
 (segment (start 70.31 58.49) (end 70.32 58.5) (width 0.25) (layer "F.Cu") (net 6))
 (segment (start 64.3082 57.12) (end 61.62 57.12) (width 0.25) (layer "F.Cu") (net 6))
 (via (at 68.453 58.49) (size 0.6) (drill 0.3) (layers "F.Cu" "B.Cu") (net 6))
 (via (at 65.659 58.4708) (size 0.6) (drill 0.3) (layers "F.Cu" "B.Cu") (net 6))
 (segment (start 68.453 58.49) (end 65.6782 58.49) (width 0.25) (layer "B.Cu") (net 6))
 (segment (start 65.6782 58.49) (end 65.659 58.4708) (width 0.25) (layer "B.Cu") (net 6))
 (segment (start 59.7916 57.2008) (end 59.7408 57.2008) (width 0.25) (layer "F.Cu") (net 5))
 (segment (start 68.472931 59.517669) (end 70.402331 59.517669) (width 0.25) (layer "F.Cu") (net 5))
 (segment (start 68.472931 59.517669) (end 68.4906 59.5) (width 0.25) (layer "F.Cu") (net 5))
 (segment (start 70.402331 59.517669) (end 70.42 59.5) (width 0.25) (layer "F.Cu") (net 5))
 (segment (start 59.7408 57.2008) (end 56.4416 60.5) (width 0.25) (layer "F.Cu") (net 5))
 (segment (start 56.4416 60.5) (end 54.98 60.5) (width 0.25) (layer "F.Cu") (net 5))
 (segment (start 68.472931 59.517669) (end 68.455262 59.5) (width 0.25) (layer "F.Cu") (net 5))
 (segment (start 70.352331 59.517669) (end 70.37 59.5) (width 0.25) (layer "F.Cu") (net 5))
 (via (at 59.7916 57.2008) (size 0.6) (drill 0.3) (layers "F.Cu" "B.Cu") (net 5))
 (via (at 68.472931 59.517669) (size 0.6) (drill 0.3) (layers "F.Cu" "B.Cu") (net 5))
 (segment (start 61.4492 57.2008) (end 59.7916 57.2008) (width 0.25) (layer "B.Cu") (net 5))
 (segment (start 68.472931 59.517669) (end 65.791469 59.517669) (width 0.25) (layer "B.Cu") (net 5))
 (segment (start 65.791469 59.517669) (end 63.4638 57.19) (width 0.25) (layer "B.Cu") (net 5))
 (segment (start 61.46 57.19) (end 61.4492 57.2008) (width 0.25) (layer "B.Cu") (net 5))
 (segment (start 63.4638 57.19) (end 61.46 57.19) (width 0.25) (layer "B.Cu") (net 5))
 (segment (start 63.627 54.4068) (end 63.1698 54.864) (width 0.25) (layer "F.Cu") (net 9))
 (segment (start 64.5202 65.881) (end 64.5202 66.081) (width 0.25) (layer "F.Cu") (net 9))
 (segment (start 62.8402 65.941) (end 62.8452 65.936) (width 0.25) (layer "F.Cu") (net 9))
 (segment (start 63.5452 65.936) (end 64.4652 65.936) (width 0.25) (layer "F.Cu") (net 9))
 (segment (start 61.6202 65.941) (end 60.4038 65.941) (width 0.25) (layer "F.Cu") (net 9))
 (segment (start 65.6082 68.5546) (end 65.1502 68.0966) (width 0.25) (layer "F.Cu") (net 9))
 (segment (start 58.55 65.1) (end 58.55 65.5858) (width 0.25) (layer "F.Cu") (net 9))
 (segment (start 62.8452 65.936) (end 63.5452 65.936) (width 0.25) (layer "F.Cu") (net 9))
 (segment (start 61.727 52.847) (end 62.1942 52.847) (width 0.25) (layer "F.Cu") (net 9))
 (segment (start 68.5546 68.5292) (end 65.6336 68.5292) (width 0.25) (layer "F.Cu") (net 9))
 (segment (start 65.1502 66.711) (end 65.1502 67.481) (width 0.25) (layer "F.Cu") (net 9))
 (segment (start 68.4754 54.6354) (end 68.83 54.99) (width 0.25) (layer "F.Cu") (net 9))
 (segment (start 63.627 53.497) (end 64.1396 53.497) (width 0.25) (layer "F.Cu") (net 9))
 (segment (start 65.278 54.6354) (end 68.4754 54.6354) (width 0.25) (layer "F.Cu") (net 9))
 (segment (start 62.1942 52.847) (end 62.8442 53.497) (width 0.25) (layer "F.Cu") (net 9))
 (segment (start 64.5202 66.081) (end 65.1502 66.711) (width 0.25) (layer "F.Cu") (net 9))
 (segment (start 61.6202 65.941) (end 62.8402 65.941) (width 0.25) (layer "F.Cu") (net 9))
 (segment (start 59.5628 65.1) (end 58.55 65.1) (width 0.25) (layer "F.Cu") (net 9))
 (segment (start 65.6336 68.5292) (end 65.6082 68.5546) (width 0.25) (layer "F.Cu") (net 9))
 (segment (start 63.627 53.497) (end 63.627 54.4068) (width 0.25) (layer "F.Cu") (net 9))
 (segment (start 64.1396 53.497) (end 65.278 54.6354) (width 0.25) (layer "F.Cu") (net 9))
 (segment (start 69.9008 67.183) (end 68.5546 68.5292) (width 0.25) (layer "F.Cu") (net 9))
 (segment (start 60.4038 65.941) (end 59.5628 65.1) (width 0.25) (layer "F.Cu") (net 9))
 (segment (start 69.9008 63.881) (end 69.9008 67.183) (width 0.25) (layer "F.Cu") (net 9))
 (segment (start 62.8442 53.497) (end 63.627 53.497) (width 0.25) (layer "F.Cu") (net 9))
 (segment (start 65.1502 68.0966) (end 65.1502 67.481) (width 0.25) (layer "F.Cu") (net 9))
 (segment (start 64.4652 65.936) (end 64.5202 65.881) (width 0.25) (layer "F.Cu") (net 9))
 (via (at 69.9008 63.881) (size 0.6) (drill 0.3) (layers "F.Cu" "B.Cu") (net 9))
 (via (at 68.83 54.99) (size 0.6) (drill 0.3) (layers "F.Cu" "B.Cu") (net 9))
 (segment (start 69.9008 56.0832) (end 68.83 55.0124) (width 0.25) (layer "B.Cu") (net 9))
 (segment (start 68.83 55.0124) (end 68.83 54.99) (width 0.25) (layer "B.Cu") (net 9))
 (segment (start 69.9008 63.881) (end 69.9008 56.0832) (width 0.25) (layer "B.Cu") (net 9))
 (segment (start 68.426 63.981) (end 68.4276 63.9826) (width 0.25) (layer "F.Cu") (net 1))
 (segment (start 66.802 61.9252) (end 66.802 63.3476) (width 0.25) (layer "F.Cu") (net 1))
 (segment (start 62.7 59.2125) (end 64.0893 59.2125) (width 0.25) (layer "F.Cu") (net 1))
 (segment (start 66.7952 63.981) (end 68.426 63.981) (width 0.25) (layer "F.Cu") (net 1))
 (segment (start 64.0893 59.2125) (end 66.802 61.9252) (width 0.25) (layer "F.Cu") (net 1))
 (segment (start 66.7952 63.3544) (end 66.7952 63.981) (width 0.25) (layer "F.Cu") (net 1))
 (segment (start 66.802 63.3476) (end 66.7952 63.3544) (width 0.25) (layer "F.Cu") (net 1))
 (segment (start 60.0375 60.7875) (end 62.7 60.7875) (width 0.25) (layer "F.Cu") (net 2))
 (segment (start 57.6 63.225) (end 57.6 62.56) (width 0.25) (layer "F.Cu") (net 2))
 (segment (start 57.6 63.225) (end 60.0375 60.7875) (width 0.25) (layer "F.Cu") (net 2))
 (segment (start 62.0058 63.225) (end 59.5 63.225) (width 0.25) (layer "F.Cu") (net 8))
 (segment (start 59.545 63.18) (end 59.5 63.225) (width 0.25) (layer "F.Cu") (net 8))
 (segment (start 64.5202 63.981) (end 62.7618 63.981) (width 0.25) (layer "F.Cu") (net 8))
 (segment (start 62.7618 63.981) (end 62.0058 63.225) (width 0.25) (layer "F.Cu") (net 8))
 (segment (start 66.7952 67.346) (end 66.6602 67.481) (width 0.25) (layer "F.Cu") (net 7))
 (segment (start 67.7164 67.3608) (end 68.4276 67.3608) (width 0.25) (layer "F.Cu") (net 7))
 (segment (start 66.7952 65.881) (end 66.7952 67.196) (width 0.25) (layer "F.Cu") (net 7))
 (segment (start 66.5226 67.481) (end 67.5962 67.481) (width 0.25) (layer "F.Cu") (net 7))
 (segment (start 66.5226 67.481) (end 66.1702 67.481) (width 0.25) (layer "F.Cu") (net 7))
 (segment (start 66.7952 67.196) (end 66.7952 67.346) (width 0.25) (layer "F.Cu") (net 7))
 (segment (start 66.6602 67.481) (end 66.5226 67.481) (width 0.25) (layer "F.Cu") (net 7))
 (segment (start 67.5962 67.481) (end 67.7164 67.3608) (width 0.25) (layer "F.Cu") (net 7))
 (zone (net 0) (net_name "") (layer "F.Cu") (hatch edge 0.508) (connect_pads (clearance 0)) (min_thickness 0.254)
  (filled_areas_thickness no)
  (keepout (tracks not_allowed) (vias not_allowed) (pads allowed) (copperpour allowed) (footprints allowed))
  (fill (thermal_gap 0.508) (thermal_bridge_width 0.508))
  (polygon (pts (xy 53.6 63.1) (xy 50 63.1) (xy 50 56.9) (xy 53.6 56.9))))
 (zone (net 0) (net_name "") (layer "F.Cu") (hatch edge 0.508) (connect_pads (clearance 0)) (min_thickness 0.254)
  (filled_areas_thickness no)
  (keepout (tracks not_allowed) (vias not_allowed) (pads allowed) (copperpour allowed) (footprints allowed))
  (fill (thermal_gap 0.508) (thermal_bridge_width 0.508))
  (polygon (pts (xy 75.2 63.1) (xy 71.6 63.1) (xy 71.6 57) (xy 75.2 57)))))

